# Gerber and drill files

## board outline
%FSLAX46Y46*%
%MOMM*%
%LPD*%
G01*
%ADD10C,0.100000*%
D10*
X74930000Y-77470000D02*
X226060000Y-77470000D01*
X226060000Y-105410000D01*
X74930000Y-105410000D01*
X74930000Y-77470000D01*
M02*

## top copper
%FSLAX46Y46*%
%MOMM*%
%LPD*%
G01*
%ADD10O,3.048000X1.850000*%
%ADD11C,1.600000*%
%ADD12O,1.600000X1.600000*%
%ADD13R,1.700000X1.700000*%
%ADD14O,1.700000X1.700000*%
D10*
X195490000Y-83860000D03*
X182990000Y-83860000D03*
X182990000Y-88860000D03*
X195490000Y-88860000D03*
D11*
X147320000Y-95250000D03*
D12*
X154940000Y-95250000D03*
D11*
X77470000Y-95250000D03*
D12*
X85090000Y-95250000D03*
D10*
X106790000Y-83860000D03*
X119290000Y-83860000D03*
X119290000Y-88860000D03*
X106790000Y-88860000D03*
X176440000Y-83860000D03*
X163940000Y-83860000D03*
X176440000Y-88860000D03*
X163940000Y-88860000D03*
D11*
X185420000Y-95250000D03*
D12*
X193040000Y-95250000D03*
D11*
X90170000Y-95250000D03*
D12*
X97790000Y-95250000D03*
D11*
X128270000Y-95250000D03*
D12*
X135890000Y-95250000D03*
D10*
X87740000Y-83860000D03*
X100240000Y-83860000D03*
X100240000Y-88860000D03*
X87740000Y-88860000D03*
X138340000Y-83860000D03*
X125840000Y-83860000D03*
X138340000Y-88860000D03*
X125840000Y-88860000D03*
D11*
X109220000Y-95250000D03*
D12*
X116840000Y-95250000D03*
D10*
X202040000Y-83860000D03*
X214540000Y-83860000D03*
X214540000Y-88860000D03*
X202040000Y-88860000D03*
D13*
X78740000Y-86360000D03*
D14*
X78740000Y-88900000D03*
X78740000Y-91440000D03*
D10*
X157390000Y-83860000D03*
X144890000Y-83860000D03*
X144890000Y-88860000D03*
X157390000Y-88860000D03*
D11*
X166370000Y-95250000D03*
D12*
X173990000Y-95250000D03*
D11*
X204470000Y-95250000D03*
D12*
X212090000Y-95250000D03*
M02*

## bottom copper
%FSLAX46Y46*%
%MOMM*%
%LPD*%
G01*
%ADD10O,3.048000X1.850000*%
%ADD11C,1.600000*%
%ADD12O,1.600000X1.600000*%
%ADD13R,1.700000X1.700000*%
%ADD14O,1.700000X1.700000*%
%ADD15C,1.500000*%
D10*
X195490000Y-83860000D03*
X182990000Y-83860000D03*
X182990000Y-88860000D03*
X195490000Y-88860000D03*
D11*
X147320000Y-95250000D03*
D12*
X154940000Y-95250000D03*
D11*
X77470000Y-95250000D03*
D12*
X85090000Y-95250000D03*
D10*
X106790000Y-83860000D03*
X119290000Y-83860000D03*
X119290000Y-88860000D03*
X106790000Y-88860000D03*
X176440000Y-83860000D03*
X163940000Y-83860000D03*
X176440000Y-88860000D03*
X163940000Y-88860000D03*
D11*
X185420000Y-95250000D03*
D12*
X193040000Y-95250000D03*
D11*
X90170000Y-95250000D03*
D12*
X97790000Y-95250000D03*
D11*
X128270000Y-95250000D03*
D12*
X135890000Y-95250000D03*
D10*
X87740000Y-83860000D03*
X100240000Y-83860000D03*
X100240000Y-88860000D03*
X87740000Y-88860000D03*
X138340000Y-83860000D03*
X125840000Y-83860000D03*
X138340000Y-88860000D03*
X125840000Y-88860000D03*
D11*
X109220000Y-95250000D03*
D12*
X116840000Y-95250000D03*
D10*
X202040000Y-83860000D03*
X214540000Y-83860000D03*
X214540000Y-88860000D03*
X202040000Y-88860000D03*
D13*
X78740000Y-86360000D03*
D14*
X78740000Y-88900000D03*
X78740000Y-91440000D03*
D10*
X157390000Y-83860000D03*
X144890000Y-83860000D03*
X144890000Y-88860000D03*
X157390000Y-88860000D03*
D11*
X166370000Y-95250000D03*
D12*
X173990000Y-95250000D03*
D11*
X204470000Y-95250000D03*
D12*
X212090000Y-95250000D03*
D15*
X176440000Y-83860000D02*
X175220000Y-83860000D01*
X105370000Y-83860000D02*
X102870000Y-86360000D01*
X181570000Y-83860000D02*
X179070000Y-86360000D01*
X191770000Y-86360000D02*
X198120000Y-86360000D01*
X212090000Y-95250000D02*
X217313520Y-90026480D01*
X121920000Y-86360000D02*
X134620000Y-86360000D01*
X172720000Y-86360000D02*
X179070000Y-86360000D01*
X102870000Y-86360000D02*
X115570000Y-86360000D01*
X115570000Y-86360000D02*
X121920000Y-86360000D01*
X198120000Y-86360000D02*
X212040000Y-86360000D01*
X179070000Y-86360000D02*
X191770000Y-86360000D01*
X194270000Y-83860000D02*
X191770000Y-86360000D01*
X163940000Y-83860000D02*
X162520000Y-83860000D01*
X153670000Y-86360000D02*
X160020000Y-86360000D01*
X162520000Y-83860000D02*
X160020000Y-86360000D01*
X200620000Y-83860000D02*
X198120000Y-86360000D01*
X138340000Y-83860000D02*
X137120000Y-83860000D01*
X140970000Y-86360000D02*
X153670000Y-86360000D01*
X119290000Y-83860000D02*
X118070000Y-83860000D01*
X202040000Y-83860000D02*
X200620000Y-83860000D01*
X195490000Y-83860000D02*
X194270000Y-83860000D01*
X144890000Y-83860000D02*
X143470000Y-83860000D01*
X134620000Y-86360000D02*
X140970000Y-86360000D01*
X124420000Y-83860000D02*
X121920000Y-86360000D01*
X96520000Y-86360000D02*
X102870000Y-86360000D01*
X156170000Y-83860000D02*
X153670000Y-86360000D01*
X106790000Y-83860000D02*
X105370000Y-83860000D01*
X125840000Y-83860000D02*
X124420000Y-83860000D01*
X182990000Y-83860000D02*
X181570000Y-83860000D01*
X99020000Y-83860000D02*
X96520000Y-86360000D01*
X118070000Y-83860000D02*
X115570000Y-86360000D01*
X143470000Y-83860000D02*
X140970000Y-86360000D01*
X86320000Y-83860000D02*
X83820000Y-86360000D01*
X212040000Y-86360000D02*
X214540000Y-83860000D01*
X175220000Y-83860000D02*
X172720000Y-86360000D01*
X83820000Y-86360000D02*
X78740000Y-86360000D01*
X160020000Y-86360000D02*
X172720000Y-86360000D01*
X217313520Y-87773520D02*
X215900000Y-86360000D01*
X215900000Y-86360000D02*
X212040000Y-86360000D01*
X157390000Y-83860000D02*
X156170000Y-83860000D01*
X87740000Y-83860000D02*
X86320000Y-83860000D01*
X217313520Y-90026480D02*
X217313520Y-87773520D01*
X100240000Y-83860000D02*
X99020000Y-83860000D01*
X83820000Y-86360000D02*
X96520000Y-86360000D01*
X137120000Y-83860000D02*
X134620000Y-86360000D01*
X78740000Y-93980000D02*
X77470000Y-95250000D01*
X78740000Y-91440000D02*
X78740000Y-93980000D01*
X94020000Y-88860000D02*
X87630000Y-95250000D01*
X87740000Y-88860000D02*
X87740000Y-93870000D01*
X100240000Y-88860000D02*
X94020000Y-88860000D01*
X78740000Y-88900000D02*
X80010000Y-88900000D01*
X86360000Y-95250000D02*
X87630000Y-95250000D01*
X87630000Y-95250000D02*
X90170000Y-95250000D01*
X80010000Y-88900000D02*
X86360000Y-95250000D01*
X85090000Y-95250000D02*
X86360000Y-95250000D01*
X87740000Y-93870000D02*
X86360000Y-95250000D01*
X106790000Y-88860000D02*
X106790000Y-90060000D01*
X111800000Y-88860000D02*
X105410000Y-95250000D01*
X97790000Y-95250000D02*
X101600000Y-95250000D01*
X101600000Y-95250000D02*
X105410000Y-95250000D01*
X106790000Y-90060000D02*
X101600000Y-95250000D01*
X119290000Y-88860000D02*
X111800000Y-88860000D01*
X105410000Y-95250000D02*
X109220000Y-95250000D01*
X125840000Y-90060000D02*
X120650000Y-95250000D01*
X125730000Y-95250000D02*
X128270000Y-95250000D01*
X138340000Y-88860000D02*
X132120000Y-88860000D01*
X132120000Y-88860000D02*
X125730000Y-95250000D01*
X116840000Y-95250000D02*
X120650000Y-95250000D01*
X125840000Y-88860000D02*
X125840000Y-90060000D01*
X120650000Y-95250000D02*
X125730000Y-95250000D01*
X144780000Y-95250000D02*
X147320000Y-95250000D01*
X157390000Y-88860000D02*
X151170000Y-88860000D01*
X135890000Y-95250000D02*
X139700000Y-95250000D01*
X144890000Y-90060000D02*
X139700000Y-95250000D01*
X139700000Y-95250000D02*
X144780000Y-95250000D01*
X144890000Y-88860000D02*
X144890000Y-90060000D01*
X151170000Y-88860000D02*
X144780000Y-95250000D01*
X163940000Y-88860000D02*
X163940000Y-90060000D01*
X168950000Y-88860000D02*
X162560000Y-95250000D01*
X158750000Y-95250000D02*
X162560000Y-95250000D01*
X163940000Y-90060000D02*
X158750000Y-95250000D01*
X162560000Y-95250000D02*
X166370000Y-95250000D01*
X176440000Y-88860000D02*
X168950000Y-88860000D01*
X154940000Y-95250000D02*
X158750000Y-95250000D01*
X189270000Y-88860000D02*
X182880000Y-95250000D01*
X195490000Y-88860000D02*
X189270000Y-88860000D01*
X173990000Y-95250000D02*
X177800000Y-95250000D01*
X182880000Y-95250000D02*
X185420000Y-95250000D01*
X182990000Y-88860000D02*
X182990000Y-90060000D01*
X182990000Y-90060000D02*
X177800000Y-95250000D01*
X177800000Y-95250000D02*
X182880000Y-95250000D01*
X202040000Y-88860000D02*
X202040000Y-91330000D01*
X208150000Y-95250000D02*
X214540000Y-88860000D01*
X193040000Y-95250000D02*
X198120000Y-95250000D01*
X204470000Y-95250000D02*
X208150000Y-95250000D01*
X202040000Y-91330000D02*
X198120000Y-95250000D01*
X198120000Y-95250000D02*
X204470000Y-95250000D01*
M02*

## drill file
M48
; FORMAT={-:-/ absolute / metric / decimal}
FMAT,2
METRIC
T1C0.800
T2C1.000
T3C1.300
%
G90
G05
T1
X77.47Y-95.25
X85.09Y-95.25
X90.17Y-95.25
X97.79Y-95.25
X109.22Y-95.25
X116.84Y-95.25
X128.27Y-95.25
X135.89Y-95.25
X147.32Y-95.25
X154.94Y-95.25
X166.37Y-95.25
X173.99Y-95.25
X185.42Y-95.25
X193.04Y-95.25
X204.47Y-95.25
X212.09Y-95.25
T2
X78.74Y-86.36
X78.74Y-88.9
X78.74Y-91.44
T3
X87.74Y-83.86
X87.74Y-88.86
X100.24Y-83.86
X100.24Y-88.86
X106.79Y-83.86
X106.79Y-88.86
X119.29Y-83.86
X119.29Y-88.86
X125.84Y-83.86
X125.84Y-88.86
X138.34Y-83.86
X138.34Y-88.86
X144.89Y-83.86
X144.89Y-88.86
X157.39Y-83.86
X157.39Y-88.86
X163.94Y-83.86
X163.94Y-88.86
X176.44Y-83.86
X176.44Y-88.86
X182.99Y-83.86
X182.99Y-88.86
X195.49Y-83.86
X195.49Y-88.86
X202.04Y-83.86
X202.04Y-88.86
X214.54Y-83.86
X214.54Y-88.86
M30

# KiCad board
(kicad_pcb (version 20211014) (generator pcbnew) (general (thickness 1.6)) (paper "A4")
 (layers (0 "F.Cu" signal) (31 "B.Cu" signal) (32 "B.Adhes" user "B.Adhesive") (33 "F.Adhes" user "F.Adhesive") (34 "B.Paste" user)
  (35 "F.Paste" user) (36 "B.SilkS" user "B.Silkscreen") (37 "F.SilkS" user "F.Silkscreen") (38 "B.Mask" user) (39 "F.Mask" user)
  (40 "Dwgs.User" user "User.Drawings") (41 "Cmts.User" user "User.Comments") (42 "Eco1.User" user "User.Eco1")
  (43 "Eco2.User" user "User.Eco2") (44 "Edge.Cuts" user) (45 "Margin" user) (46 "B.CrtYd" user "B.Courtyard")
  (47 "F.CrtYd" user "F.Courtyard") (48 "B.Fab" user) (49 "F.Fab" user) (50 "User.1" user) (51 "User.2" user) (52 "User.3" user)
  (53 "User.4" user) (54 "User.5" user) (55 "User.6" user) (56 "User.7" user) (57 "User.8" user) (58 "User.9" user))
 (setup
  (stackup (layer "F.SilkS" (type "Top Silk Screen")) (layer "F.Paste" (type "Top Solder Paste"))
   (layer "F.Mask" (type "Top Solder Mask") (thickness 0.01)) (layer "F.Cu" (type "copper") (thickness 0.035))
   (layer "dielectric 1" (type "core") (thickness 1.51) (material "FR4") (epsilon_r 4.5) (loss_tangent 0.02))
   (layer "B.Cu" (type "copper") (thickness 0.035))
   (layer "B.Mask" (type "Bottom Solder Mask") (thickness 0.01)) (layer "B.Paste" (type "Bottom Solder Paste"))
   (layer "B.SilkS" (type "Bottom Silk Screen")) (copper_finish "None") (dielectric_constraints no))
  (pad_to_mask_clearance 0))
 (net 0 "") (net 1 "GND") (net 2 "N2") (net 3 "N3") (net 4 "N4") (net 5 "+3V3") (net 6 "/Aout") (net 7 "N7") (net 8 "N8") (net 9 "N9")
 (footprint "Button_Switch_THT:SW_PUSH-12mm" (layer "F.Cu") (at 182.99 83.86)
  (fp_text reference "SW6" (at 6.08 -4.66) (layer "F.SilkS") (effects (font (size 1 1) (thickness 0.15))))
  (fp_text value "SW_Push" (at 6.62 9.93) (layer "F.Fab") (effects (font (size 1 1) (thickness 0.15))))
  (pad "1" thru_hole oval (at 12.5 0) (size 3.048 1.85) (drill 1.3) (layers *.Cu *.Mask) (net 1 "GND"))
  (pad "1" thru_hole oval (at 0 0) (size 3.048 1.85) (drill 1.3) (layers *.Cu *.Mask) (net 1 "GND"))
  (pad "2" thru_hole oval (at 0 5) (size 3.048 1.85) (drill 1.3) (layers *.Cu *.Mask) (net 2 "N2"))
  (pad "2" thru_hole oval (at 12.5 5) (size 3.048 1.85) (drill 1.3) (layers *.Cu *.Mask) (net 2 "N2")))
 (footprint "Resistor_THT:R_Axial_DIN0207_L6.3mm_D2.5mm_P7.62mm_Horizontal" (layer "F.Cu") (at 147.32 95.25)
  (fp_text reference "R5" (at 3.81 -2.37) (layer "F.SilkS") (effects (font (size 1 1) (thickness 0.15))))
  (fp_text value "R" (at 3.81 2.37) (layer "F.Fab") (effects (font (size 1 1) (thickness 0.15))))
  (pad "1" thru_hole circle (at 0 0) (size 1.6 1.6) (drill 0.8) (layers *.Cu *.Mask) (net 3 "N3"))
  (pad "2" thru_hole oval (at 7.62 0) (size 1.6 1.6) (drill 0.8) (layers *.Cu *.Mask) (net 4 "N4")))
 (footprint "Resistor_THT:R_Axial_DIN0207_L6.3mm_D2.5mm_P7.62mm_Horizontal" (layer "F.Cu") (at 77.47 95.25)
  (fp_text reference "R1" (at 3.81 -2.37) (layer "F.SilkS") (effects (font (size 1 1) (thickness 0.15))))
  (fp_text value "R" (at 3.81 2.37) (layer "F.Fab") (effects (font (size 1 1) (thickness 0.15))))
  (pad "1" thru_hole circle (at 0 0) (size 1.6 1.6) (drill 0.8) (layers *.Cu *.Mask) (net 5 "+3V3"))
  (pad "2" thru_hole oval (at 7.62 0) (size 1.6 1.6) (drill 0.8) (layers *.Cu *.Mask) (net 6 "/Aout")))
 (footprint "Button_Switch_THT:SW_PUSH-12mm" (layer "F.Cu") (at 106.79 83.86)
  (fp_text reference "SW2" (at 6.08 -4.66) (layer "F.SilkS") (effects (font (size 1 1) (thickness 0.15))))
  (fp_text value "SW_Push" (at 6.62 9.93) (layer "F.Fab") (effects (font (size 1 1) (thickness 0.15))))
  (pad "1" thru_hole oval (at 0 0) (size 3.048 1.85) (drill 1.3) (layers *.Cu *.Mask) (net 1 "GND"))
  (pad "1" thru_hole oval (at 12.5 0) (size 3.048 1.85) (drill 1.3) (layers *.Cu *.Mask) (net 1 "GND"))
  (pad "2" thru_hole oval (at 12.5 5) (size 3.048 1.85) (drill 1.3) (layers *.Cu *.Mask) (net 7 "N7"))
  (pad "2" thru_hole oval (at 0 5) (size 3.048 1.85) (drill 1.3) (layers *.Cu *.Mask) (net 7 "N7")))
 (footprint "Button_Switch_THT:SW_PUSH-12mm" (layer "F.Cu") (at 163.94 83.86)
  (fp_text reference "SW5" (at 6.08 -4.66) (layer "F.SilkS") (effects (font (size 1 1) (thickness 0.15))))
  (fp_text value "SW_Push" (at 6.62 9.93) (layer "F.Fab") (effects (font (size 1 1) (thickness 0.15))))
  (pad "1" thru_hole oval (at 12.5 0) (size 3.048 1.85) (drill 1.3) (layers *.Cu *.Mask) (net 1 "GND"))
  (pad "1" thru_hole oval (at 0 0) (size 3.048 1.85) (drill 1.3) (layers *.Cu *.Mask) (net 1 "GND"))
  (pad "2" thru_hole oval (at 12.5 5) (size 3.048 1.85) (drill 1.3) (layers *.Cu *.Mask) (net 4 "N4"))
  (pad "2" thru_hole oval (at 0 5) (size 3.048 1.85) (drill 1.3) (layers *.Cu *.Mask) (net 4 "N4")))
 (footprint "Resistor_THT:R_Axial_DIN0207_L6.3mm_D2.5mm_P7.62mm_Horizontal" (layer "F.Cu") (at 185.42 95.25)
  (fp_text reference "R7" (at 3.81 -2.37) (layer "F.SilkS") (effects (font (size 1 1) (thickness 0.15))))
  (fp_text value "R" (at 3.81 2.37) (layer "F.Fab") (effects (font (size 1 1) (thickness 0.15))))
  (pad "1" thru_hole circle (at 0 0) (size 1.6 1.6) (drill 0.8) (layers *.Cu *.Mask) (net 2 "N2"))
  (pad "2" thru_hole oval (at 7.62 0) (size 1.6 1.6) (drill 0.8) (layers *.Cu *.Mask) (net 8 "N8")))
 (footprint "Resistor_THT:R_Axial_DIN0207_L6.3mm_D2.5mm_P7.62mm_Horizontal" (layer "F.Cu") (at 90.17 95.25)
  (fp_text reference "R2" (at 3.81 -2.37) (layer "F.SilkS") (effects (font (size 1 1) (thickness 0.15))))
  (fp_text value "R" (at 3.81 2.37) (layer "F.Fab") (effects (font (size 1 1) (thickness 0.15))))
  (pad "1" thru_hole circle (at 0 0) (size 1.6 1.6) (drill 0.8) (layers *.Cu *.Mask) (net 6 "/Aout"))
  (pad "2" thru_hole oval (at 7.62 0) (size 1.6 1.6) (drill 0.8) (layers *.Cu *.Mask) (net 7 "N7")))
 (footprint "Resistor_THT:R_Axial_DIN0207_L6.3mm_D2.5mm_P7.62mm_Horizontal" (layer "F.Cu") (at 128.27 95.25)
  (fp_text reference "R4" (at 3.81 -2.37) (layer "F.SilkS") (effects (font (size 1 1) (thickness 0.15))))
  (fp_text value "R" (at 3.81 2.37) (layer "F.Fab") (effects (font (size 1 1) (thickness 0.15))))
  (pad "1" thru_hole circle (at 0 0) (size 1.6 1.6) (drill 0.8) (layers *.Cu *.Mask) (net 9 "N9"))
  (pad "2" thru_hole oval (at 7.62 0) (size 1.6 1.6) (drill 0.8) (layers *.Cu *.Mask) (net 3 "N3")))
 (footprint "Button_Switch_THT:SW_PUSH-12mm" (layer "F.Cu") (at 87.74 83.86)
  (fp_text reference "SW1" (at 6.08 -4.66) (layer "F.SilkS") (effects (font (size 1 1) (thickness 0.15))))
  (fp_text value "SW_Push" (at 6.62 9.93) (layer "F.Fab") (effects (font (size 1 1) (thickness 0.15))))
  (pad "1" thru_hole oval (at 0 0) (size 3.048 1.85) (drill 1.3) (layers *.Cu *.Mask) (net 1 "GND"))
  (pad "1" thru_hole oval (at 12.5 0) (size 3.048 1.85) (drill 1.3) (layers *.Cu *.Mask) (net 1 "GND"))
  (pad "2" thru_hole oval (at 12.5 5) (size 3.048 1.85) (drill 1.3) (layers *.Cu *.Mask) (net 6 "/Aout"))
  (pad "2" thru_hole oval (at 0 5) (size 3.048 1.85) (drill 1.3) (layers *.Cu *.Mask) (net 6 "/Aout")))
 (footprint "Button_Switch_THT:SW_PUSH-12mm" (layer "F.Cu") (at 125.84 83.86)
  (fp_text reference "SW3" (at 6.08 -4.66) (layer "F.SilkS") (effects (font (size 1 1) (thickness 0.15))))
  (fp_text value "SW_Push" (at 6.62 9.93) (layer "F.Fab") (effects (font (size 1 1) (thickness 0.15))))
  (pad "1" thru_hole oval (at 12.5 0) (size 3.048 1.85) (drill 1.3) (layers *.Cu *.Mask) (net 1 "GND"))
  (pad "1" thru_hole oval (at 0 0) (size 3.048 1.85) (drill 1.3) (layers *.Cu *.Mask) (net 1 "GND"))
  (pad "2" thru_hole oval (at 12.5 5) (size 3.048 1.85) (drill 1.3) (layers *.Cu *.Mask) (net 9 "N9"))
  (pad "2" thru_hole oval (at 0 5) (size 3.048 1.85) (drill 1.3) (layers *.Cu *.Mask) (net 9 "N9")))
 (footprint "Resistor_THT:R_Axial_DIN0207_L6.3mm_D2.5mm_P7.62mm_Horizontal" (layer "F.Cu") (at 109.22 95.25)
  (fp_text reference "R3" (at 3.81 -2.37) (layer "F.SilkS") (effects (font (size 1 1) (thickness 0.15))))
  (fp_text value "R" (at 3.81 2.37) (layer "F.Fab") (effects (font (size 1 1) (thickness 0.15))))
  (pad "1" thru_hole circle (at 0 0) (size 1.6 1.6) (drill 0.8) (layers *.Cu *.Mask) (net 7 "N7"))
  (pad "2" thru_hole oval (at 7.62 0) (size 1.6 1.6) (drill 0.8) (layers *.Cu *.Mask) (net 9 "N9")))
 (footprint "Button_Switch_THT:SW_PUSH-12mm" (layer "F.Cu") (at 202.04 83.86)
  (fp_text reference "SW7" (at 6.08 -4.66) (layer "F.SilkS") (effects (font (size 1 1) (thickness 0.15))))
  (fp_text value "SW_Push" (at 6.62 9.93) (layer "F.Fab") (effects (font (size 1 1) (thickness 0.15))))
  (pad "1" thru_hole oval (at 0 0) (size 3.048 1.85) (drill 1.3) (layers *.Cu *.Mask) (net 1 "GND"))
  (pad "1" thru_hole oval (at 12.5 0) (size 3.048 1.85) (drill 1.3) (layers *.Cu *.Mask) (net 1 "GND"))
  (pad "2" thru_hole oval (at 12.5 5) (size 3.048 1.85) (drill 1.3) (layers *.Cu *.Mask) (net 8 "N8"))
  (pad "2" thru_hole oval (at 0 5) (size 3.048 1.85) (drill 1.3) (layers *.Cu *.Mask) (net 8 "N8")))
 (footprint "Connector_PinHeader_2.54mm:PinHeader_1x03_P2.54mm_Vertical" (layer "F.Cu") (at 78.74 86.36)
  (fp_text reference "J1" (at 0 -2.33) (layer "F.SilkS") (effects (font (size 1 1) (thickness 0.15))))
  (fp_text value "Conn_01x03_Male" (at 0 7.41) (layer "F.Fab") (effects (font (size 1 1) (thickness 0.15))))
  (pad "1" thru_hole rect (at 0 0) (size 1.7 1.7) (drill 1) (layers *.Cu *.Mask) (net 1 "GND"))
  (pad "2" thru_hole oval (at 0 2.54) (size 1.7 1.7) (drill 1) (layers *.Cu *.Mask) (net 6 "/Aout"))
  (pad "3" thru_hole oval (at 0 5.08) (size 1.7 1.7) (drill 1) (layers *.Cu *.Mask) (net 5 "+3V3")))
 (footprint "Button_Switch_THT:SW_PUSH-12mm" (layer "F.Cu") (at 144.89 83.86)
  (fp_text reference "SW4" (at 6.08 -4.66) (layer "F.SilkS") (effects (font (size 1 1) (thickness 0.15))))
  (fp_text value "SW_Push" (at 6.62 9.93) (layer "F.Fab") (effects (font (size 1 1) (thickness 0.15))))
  (pad "1" thru_hole oval (at 12.5 0) (size 3.048 1.85) (drill 1.3) (layers *.Cu *.Mask) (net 1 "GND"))
  (pad "1" thru_hole oval (at 0 0) (size 3.048 1.85) (drill 1.3) (layers *.Cu *.Mask) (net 1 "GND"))
  (pad "2" thru_hole oval (at 0 5) (size 3.048 1.85) (drill 1.3) (layers *.Cu *.Mask) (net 3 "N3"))
  (pad "2" thru_hole oval (at 12.5 5) (size 3.048 1.85) (drill 1.3) (layers *.Cu *.Mask) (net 3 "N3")))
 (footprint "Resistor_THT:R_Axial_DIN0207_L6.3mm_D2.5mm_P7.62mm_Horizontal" (layer "F.Cu") (at 166.37 95.25)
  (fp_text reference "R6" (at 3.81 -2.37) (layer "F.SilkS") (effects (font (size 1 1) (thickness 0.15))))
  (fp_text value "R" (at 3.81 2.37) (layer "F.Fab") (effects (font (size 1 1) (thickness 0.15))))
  (pad "1" thru_hole circle (at 0 0) (size 1.6 1.6) (drill 0.8) (layers *.Cu *.Mask) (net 4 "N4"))
  (pad "2" thru_hole oval (at 7.62 0) (size 1.6 1.6) (drill 0.8) (layers *.Cu *.Mask) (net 2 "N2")))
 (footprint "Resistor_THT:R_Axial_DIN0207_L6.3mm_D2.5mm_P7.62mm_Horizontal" (layer "F.Cu") (at 204.47 95.25)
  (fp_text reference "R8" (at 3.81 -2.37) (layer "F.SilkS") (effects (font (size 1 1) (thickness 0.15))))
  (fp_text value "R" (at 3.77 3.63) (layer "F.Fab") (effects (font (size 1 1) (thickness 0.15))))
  (pad "1" thru_hole circle (at 0 0) (size 1.6 1.6) (drill 0.8) (layers *.Cu *.Mask) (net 8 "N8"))
  (pad "2" thru_hole oval (at 7.62 0) (size 1.6 1.6) (drill 0.8) (layers *.Cu *.Mask) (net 1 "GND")))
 (gr_rect (start 74.93 77.47) (end 226.06 105.41) (layer "Edge.Cuts") (width 0.1) (fill none))
 (segment (start 176.44 83.86) (end 175.22 83.86) (width 1.5) (layer "B.Cu") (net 1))
 (segment (start 105.37 83.86) (end 102.87 86.36) (width 1.5) (layer "B.Cu") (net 1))
 (segment (start 181.57 83.86) (end 179.07 86.36) (width 1.5) (layer "B.Cu") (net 1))
 (segment (start 191.77 86.36) (end 198.12 86.36) (width 1.5) (layer "B.Cu") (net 1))
 (segment (start 212.09 95.25) (end 217.31352 90.02648) (width 1.5) (layer "B.Cu") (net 1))
 (segment (start 121.92 86.36) (end 134.62 86.36) (width 1.5) (layer "B.Cu") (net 1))
 (segment (start 172.72 86.36) (end 179.07 86.36) (width 1.5) (layer "B.Cu") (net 1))
 (segment (start 102.87 86.36) (end 115.57 86.36) (width 1.5) (layer "B.Cu") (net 1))
 (segment (start 115.57 86.36) (end 121.92 86.36) (width 1.5) (layer "B.Cu") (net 1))
 (segment (start 198.12 86.36) (end 212.04 86.36) (width 1.5) (layer "B.Cu") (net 1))
 (segment (start 179.07 86.36) (end 191.77 86.36) (width 1.5) (layer "B.Cu") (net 1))
 (segment (start 194.27 83.86) (end 191.77 86.36) (width 1.5) (layer "B.Cu") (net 1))
 (segment (start 163.94 83.86) (end 162.52 83.86) (width 1.5) (layer "B.Cu") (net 1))
 (segment (start 153.67 86.36) (end 160.02 86.36) (width 1.5) (layer "B.Cu") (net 1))
 (segment (start 162.52 83.86) (end 160.02 86.36) (width 1.5) (layer "B.Cu") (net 1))
 (segment (start 200.62 83.86) (end 198.12 86.36) (width 1.5) (layer "B.Cu") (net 1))
 (segment (start 138.34 83.86) (end 137.12 83.86) (width 1.5) (layer "B.Cu") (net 1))
 (segment (start 140.97 86.36) (end 153.67 86.36) (width 1.5) (layer "B.Cu") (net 1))
 (segment (start 119.29 83.86) (end 118.07 83.86) (width 1.5) (layer "B.Cu") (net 1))
 (segment (start 202.04 83.86) (end 200.62 83.86) (width 1.5) (layer "B.Cu") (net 1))
 (segment (start 195.49 83.86) (end 194.27 83.86) (width 1.5) (layer "B.Cu") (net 1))
 (segment (start 144.89 83.86) (end 143.47 83.86) (width 1.5) (layer "B.Cu") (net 1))
 (segment (start 134.62 86.36) (end 140.97 86.36) (width 1.5) (layer "B.Cu") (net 1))
 (segment (start 124.42 83.86) (end 121.92 86.36) (width 1.5) (layer "B.Cu") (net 1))
 (segment (start 96.52 86.36) (end 102.87 86.36) (width 1.5) (layer "B.Cu") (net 1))
 (segment (start 156.17 83.86) (end 153.67 86.36) (width 1.5) (layer "B.Cu") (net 1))
 (segment (start 106.79 83.86) (end 105.37 83.86) (width 1.5) (layer "B.Cu") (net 1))
 (segment (start 125.84 83.86) (end 124.42 83.86) (width 1.5) (layer "B.Cu") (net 1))
 (segment (start 182.99 83.86) (end 181.57 83.86) (width 1.5) (layer "B.Cu") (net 1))
 (segment (start 99.02 83.86) (end 96.52 86.36) (width 1.5) (layer "B.Cu") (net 1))
 (segment (start 118.07 83.86) (end 115.57 86.36) (width 1.5) (layer "B.Cu") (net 1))
 (segment (start 143.47 83.86) (end 140.97 86.36) (width 1.5) (layer "B.Cu") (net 1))
 (segment (start 86.32 83.86) (end 83.82 86.36) (width 1.5) (layer "B.Cu") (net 1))
 (segment (start 212.04 86.36) (end 214.54 83.86) (width 1.5) (layer "B.Cu") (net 1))
 (segment (start 175.22 83.86) (end 172.72 86.36) (width 1.5) (layer "B.Cu") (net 1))
 (segment (start 83.82 86.36) (end 78.74 86.36) (width 1.5) (layer "B.Cu") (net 1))
 (segment (start 160.02 86.36) (end 172.72 86.36) (width 1.5) (layer "B.Cu") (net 1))
 (segment (start 217.31352 87.77352) (end 215.9 86.36) (width 1.5) (layer "B.Cu") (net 1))
 (segment (start 215.9 86.36) (end 212.04 86.36) (width 1.5) (layer "B.Cu") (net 1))
 (segment (start 157.39 83.86) (end 156.17 83.86) (width 1.5) (layer "B.Cu") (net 1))
 (segment (start 87.74 83.86) (end 86.32 83.86) (width 1.5) (layer "B.Cu") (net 1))
 (segment (start 217.31352 90.02648) (end 217.31352 87.77352) (width 1.5) (layer "B.Cu") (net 1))
 (segment (start 100.24 83.86) (end 99.02 83.86) (width 1.5) (layer "B.Cu") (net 1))
 (segment (start 83.82 86.36) (end 96.52 86.36) (width 1.5) (layer "B.Cu") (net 1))
 (segment (start 137.12 83.86) (end 134.62 86.36) (width 1.5) (layer "B.Cu") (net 1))
 (segment (start 78.74 93.98) (end 77.47 95.25) (width 1.5) (layer "B.Cu") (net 5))
 (segment (start 78.74 91.44) (end 78.74 93.98) (width 1.5) (layer "B.Cu") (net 5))
 (segment (start 94.02 88.86) (end 87.63 95.25) (width 1.5) (layer "B.Cu") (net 6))
 (segment (start 87.74 88.86) (end 87.74 93.87) (width 1.5) (layer "B.Cu") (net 6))
 (segment (start 100.24 88.86) (end 94.02 88.86) (width 1.5) (layer "B.Cu") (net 6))
 (segment (start 78.74 88.9) (end 80.01 88.9) (width 1.5) (layer "B.Cu") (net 6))
 (segment (start 86.36 95.25) (end 87.63 95.25) (width 1.5) (layer "B.Cu") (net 6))
 (segment (start 87.63 95.25) (end 90.17 95.25) (width 1.5) (layer "B.Cu") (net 6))
 (segment (start 80.01 88.9) (end 86.36 95.25) (width 1.5) (layer "B.Cu") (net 6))
 (segment (start 85.09 95.25) (end 86.36 95.25) (width 1.5) (layer "B.Cu") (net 6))
 (segment (start 87.74 93.87) (end 86.36 95.25) (width 1.5) (layer "B.Cu") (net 6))
 (segment (start 106.79 88.86) (end 106.79 90.06) (width 1.5) (layer "B.Cu") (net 7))
 (segment (start 111.8 88.86) (end 105.41 95.25) (width 1.5) (layer "B.Cu") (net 7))
 (segment (start 97.79 95.25) (end 101.6 95.25) (width 1.5) (layer "B.Cu") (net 7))
 (segment (start 101.6 95.25) (end 105.41 95.25) (width 1.5) (layer "B.Cu") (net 7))
 (segment (start 106.79 90.06) (end 101.6 95.25) (width 1.5) (layer "B.Cu") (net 7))
 (segment (start 119.29 88.86) (end 111.8 88.86) (width 1.5) (layer "B.Cu") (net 7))
 (segment (start 105.41 95.25) (end 109.22 95.25) (width 1.5) (layer "B.Cu") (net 7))
 (segment (start 125.84 90.06) (end 120.65 95.25) (width 1.5) (layer "B.Cu") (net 9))
 (segment (start 125.73 95.25) (end 128.27 95.25) (width 1.5) (layer "B.Cu") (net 9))
 (segment (start 138.34 88.86) (end 132.12 88.86) (width 1.5) (layer "B.Cu") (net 9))
 (segment (start 132.12 88.86) (end 125.73 95.25) (width 1.5) (layer "B.Cu") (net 9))
 (segment (start 116.84 95.25) (end 120.65 95.25) (width 1.5) (layer "B.Cu") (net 9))
 (segment (start 125.84 88.86) (end 125.84 90.06) (width 1.5) (layer "B.Cu") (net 9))
 (segment (start 120.65 95.25) (end 125.73 95.25) (width 1.5) (layer "B.Cu") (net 9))
 (segment (start 144.78 95.25) (end 147.32 95.25) (width 1.5) (layer "B.Cu") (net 3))
 (segment (start 157.39 88.86) (end 151.17 88.86) (width 1.5) (layer "B.Cu") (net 3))
 (segment (start 135.89 95.25) (end 139.7 95.25) (width 1.5) (layer "B.Cu") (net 3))
 (segment (start 144.89 90.06) (end 139.7 95.25) (width 1.5) (layer "B.Cu") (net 3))
 (segment (start 139.7 95.25) (end 144.78 95.25) (width 1.5) (layer "B.Cu") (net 3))
 (segment (start 144.89 88.86) (end 144.89 90.06) (width 1.5) (layer "B.Cu") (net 3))
 (segment (start 151.17 88.86) (end 144.78 95.25) (width 1.5) (layer "B.Cu") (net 3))
 (segment (start 163.94 88.86) (end 163.94 90.06) (width 1.5) (layer "B.Cu") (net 4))
 (segment (start 168.95 88.86) (end 162.56 95.25) (width 1.5) (layer "B.Cu") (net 4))
 (segment (start 158.75 95.25) (end 162.56 95.25) (width 1.5) (layer "B.Cu") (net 4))
 (segment (start 163.94 90.06) (end 158.75 95.25) (width 1.5) (layer "B.Cu") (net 4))
 (segment (start 162.56 95.25) (end 166.37 95.25) (width 1.5) (layer "B.Cu") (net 4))
 (segment (start 176.44 88.86) (end 168.95 88.86) (width 1.5) (layer "B.Cu") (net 4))
 (segment (start 154.94 95.25) (end 158.75 95.25) (width 1.5) (layer "B.Cu") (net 4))
 (segment (start 189.27 88.86) (end 182.88 95.25) (width 1.5) (layer "B.Cu") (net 2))
 (segment (start 195.49 88.86) (end 189.27 88.86) (width 1.5) (layer "B.Cu") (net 2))
 (segment (start 173.99 95.25) (end 177.8 95.25) (width 1.5) (layer "B.Cu") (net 2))
 (segment (start 182.88 95.25) (end 185.42 95.25) (width 1.5) (layer "B.Cu") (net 2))
 (segment (start 182.99 88.86) (end 182.99 90.06) (width 1.5) (layer "B.Cu") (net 2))
 (segment (start 182.99 90.06) (end 177.8 95.25) (width 1.5) (layer "B.Cu") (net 2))
 (segment (start 177.8 95.25) (end 182.88 95.25) (width 1.5) (layer "B.Cu") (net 2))
 (segment (start 202.04 88.86) (end 202.04 91.33) (width 1.5) (layer "B.Cu") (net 8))
 (segment (start 208.15 95.25) (end 214.54 88.86) (width 1.5) (layer "B.Cu") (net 8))
 (segment (start 193.04 95.25) (end 198.12 95.25) (width 1.5) (layer "B.Cu") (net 8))
 (segment (start 204.47 95.25) (end 208.15 95.25) (width 1.5) (layer "B.Cu") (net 8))
 (segment (start 202.04 91.33) (end 198.12 95.25) (width 1.5) (layer "B.Cu") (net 8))
 (segment (start 198.12 95.25) (end 204.47 95.25) (width 1.5) (layer "B.Cu") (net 8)))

